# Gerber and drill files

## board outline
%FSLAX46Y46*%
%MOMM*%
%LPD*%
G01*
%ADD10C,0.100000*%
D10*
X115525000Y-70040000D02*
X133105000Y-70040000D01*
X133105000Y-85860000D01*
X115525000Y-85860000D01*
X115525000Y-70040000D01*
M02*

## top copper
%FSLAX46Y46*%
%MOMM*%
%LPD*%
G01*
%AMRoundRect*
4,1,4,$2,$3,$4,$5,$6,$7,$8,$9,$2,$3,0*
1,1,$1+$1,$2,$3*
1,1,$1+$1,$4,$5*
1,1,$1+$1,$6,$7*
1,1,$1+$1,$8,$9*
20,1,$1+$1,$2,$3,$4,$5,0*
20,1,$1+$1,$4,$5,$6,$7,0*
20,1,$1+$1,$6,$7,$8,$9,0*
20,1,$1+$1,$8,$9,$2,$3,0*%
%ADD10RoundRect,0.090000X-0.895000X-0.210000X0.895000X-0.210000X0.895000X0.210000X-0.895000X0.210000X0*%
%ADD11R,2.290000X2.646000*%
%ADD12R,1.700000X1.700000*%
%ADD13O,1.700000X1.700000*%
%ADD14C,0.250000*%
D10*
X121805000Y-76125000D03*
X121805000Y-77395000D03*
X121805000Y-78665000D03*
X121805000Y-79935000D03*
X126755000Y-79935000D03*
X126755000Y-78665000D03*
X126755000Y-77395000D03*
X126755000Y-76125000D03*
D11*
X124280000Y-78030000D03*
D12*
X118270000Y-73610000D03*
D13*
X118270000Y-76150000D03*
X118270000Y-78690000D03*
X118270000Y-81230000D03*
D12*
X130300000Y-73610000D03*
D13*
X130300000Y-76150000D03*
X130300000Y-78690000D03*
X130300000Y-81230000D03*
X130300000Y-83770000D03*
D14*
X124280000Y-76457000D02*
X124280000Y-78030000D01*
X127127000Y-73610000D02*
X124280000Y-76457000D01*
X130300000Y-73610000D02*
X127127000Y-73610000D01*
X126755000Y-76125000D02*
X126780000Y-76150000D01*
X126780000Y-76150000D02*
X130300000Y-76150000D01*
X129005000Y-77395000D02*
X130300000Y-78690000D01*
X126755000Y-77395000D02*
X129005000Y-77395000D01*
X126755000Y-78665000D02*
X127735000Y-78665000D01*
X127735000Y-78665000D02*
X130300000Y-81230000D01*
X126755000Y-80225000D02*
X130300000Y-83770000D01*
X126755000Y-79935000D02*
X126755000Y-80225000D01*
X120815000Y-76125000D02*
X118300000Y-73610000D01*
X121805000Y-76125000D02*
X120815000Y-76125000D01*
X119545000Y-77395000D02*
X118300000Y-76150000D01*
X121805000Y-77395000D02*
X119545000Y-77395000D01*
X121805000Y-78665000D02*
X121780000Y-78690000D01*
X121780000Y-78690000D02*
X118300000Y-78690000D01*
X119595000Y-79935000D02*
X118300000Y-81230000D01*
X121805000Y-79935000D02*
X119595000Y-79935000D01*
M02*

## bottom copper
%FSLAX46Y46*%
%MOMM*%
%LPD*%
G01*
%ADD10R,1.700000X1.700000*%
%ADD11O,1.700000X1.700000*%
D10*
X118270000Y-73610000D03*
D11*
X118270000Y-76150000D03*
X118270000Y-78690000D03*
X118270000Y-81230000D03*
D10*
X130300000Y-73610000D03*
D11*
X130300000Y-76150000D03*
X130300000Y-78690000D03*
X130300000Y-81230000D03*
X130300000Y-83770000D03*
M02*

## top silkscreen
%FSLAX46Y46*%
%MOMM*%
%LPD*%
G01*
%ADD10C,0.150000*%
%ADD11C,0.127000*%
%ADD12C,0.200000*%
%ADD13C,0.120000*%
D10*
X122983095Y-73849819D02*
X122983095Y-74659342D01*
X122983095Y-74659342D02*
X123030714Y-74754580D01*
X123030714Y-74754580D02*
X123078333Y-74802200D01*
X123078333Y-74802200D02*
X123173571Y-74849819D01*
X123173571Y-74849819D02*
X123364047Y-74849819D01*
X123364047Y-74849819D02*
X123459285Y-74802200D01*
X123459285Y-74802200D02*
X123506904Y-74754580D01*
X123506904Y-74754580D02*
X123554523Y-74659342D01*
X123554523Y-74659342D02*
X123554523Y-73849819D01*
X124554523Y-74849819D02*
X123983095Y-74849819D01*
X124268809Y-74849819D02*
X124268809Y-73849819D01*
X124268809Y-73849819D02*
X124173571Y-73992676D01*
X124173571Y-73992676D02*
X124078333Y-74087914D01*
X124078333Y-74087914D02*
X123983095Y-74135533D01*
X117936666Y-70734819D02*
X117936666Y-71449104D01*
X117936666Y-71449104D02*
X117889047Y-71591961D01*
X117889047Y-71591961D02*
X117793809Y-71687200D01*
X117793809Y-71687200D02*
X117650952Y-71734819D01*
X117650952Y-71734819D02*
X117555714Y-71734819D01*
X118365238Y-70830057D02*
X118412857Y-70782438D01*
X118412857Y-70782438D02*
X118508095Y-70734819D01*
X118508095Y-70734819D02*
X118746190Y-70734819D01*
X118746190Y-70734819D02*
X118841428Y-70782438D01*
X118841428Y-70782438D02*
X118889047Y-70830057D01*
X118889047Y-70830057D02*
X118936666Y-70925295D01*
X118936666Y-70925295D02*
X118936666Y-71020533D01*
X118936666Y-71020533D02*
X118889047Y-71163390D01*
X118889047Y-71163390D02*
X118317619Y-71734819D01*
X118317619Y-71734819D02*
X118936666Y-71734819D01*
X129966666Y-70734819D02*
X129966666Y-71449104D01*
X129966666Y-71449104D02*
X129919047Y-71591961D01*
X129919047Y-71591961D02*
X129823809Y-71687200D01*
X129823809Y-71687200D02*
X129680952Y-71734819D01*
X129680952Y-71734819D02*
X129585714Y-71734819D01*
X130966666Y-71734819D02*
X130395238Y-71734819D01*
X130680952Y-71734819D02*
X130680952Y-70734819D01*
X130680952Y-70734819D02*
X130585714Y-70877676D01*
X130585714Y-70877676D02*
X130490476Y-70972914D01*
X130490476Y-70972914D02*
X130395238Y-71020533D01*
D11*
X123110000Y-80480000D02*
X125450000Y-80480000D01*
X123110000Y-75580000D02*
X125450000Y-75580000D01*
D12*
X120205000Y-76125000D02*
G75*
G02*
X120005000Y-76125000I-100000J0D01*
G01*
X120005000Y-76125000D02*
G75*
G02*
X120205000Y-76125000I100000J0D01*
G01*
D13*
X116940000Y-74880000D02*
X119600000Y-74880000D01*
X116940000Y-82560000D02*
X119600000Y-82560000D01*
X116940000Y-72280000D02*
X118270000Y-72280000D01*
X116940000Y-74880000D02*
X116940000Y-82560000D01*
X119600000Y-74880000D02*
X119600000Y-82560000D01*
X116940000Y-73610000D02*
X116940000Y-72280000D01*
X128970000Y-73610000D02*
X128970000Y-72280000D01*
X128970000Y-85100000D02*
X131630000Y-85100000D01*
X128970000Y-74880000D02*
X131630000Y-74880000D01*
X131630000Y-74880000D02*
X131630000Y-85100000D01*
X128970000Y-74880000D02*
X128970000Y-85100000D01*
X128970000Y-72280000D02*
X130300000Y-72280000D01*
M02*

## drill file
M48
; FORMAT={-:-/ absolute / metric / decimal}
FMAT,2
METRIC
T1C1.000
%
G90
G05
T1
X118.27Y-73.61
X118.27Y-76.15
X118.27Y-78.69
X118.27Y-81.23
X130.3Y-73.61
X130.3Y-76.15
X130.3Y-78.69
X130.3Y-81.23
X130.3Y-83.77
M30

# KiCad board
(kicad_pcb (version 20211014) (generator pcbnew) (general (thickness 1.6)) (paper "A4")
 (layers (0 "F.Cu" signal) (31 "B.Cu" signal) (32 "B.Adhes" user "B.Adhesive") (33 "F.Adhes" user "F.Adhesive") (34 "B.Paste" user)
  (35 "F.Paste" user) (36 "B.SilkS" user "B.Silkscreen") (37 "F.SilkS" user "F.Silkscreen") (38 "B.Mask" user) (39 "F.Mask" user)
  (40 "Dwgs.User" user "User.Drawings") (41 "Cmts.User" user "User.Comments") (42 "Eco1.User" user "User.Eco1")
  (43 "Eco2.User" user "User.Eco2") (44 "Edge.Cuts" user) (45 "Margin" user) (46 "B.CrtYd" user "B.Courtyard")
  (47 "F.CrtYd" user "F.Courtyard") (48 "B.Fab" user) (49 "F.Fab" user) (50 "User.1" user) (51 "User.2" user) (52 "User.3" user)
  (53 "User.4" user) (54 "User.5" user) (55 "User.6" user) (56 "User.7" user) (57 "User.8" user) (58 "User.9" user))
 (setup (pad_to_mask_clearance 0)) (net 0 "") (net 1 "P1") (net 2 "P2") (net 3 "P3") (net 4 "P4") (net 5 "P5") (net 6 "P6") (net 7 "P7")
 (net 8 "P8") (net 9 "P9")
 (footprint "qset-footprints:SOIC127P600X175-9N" (layer "F.Cu") (at 124.28 78.03)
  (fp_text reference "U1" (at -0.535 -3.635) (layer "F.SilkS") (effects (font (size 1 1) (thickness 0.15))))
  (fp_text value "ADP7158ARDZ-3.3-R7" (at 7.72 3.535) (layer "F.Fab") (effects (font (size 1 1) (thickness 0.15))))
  (fp_line (start -1.17 2.45) (end 1.17 2.45) (layer "F.SilkS") (width 0.127))
  (fp_line (start -1.17 -2.45) (end 1.17 -2.45) (layer "F.SilkS") (width 0.127))
  (fp_circle (center -4.175 -1.905) (end -4.075 -1.905) (layer "F.SilkS") (width 0.2) (fill none))
  (pad "1" smd roundrect locked (at -2.475 -1.905) (size 1.97 0.6) (layers "F.Cu" "F.Paste" "F.Mask") (roundrect_rratio 0.15) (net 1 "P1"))
  (pad "2" smd roundrect locked (at -2.475 -0.635) (size 1.97 0.6) (layers "F.Cu" "F.Paste" "F.Mask") (roundrect_rratio 0.15) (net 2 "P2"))
  (pad "3" smd roundrect locked (at -2.475 0.635) (size 1.97 0.6) (layers "F.Cu" "F.Paste" "F.Mask") (roundrect_rratio 0.15) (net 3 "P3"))
  (pad "4" smd roundrect locked (at -2.475 1.905) (size 1.97 0.6) (layers "F.Cu" "F.Paste" "F.Mask") (roundrect_rratio 0.15) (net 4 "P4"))
  (pad "5" smd roundrect locked (at 2.475 1.905) (size 1.97 0.6) (layers "F.Cu" "F.Paste" "F.Mask") (roundrect_rratio 0.15) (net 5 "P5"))
  (pad "6" smd roundrect locked (at 2.475 0.635) (size 1.97 0.6) (layers "F.Cu" "F.Paste" "F.Mask") (roundrect_rratio 0.15) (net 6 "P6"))
  (pad "7" smd roundrect locked (at 2.475 -0.635) (size 1.97 0.6) (layers "F.Cu" "F.Paste" "F.Mask") (roundrect_rratio 0.15) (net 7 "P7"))
  (pad "8" smd roundrect locked (at 2.475 -1.905) (size 1.97 0.6) (layers "F.Cu" "F.Paste" "F.Mask") (roundrect_rratio 0.15) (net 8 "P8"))
  (pad "9" smd rect locked (at 0 0) (size 2.29 2.646) (layers "F.Cu" "F.Paste" "F.Mask") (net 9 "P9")))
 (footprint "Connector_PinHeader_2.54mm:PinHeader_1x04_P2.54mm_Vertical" (layer "F.Cu") (at 118.27 73.61)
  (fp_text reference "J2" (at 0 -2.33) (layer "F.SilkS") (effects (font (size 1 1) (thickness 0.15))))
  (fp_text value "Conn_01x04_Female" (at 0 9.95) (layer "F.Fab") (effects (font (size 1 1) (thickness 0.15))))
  (fp_line (start -1.33 1.27) (end 1.33 1.27) (layer "F.SilkS") (width 0.12))
  (fp_line (start -1.33 8.95) (end 1.33 8.95) (layer "F.SilkS") (width 0.12))
  (fp_line (start -1.33 -1.33) (end 0 -1.33) (layer "F.SilkS") (width 0.12))
  (fp_line (start -1.33 1.27) (end -1.33 8.95) (layer "F.SilkS") (width 0.12))
  (fp_line (start 1.33 1.27) (end 1.33 8.95) (layer "F.SilkS") (width 0.12))
  (fp_line (start -1.33 0) (end -1.33 -1.33) (layer "F.SilkS") (width 0.12))
  (pad "1" thru_hole rect (at 0 0) (size 1.7 1.7) (drill 1) (layers *.Cu *.Mask) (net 1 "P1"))
  (pad "2" thru_hole oval (at 0 2.54) (size 1.7 1.7) (drill 1) (layers *.Cu *.Mask) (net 2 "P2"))
  (pad "3" thru_hole oval (at 0 5.08) (size 1.7 1.7) (drill 1) (layers *.Cu *.Mask) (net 3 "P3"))
  (pad "4" thru_hole oval (at 0 7.62) (size 1.7 1.7) (drill 1) (layers *.Cu *.Mask) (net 4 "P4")))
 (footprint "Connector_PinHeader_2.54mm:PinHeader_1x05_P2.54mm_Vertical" (layer "F.Cu") (at 130.3 73.61)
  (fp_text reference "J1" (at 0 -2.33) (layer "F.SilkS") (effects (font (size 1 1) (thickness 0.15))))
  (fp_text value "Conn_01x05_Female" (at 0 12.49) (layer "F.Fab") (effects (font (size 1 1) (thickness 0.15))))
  (fp_line (start -1.33 0) (end -1.33 -1.33) (layer "F.SilkS") (width 0.12))
  (fp_line (start -1.33 11.49) (end 1.33 11.49) (layer "F.SilkS") (width 0.12))
  (fp_line (start -1.33 1.27) (end 1.33 1.27) (layer "F.SilkS") (width 0.12))
  (fp_line (start 1.33 1.27) (end 1.33 11.49) (layer "F.SilkS") (width 0.12))
  (fp_line (start -1.33 1.27) (end -1.33 11.49) (layer "F.SilkS") (width 0.12))
  (fp_line (start -1.33 -1.33) (end 0 -1.33) (layer "F.SilkS") (width 0.12))
  (pad "1" thru_hole rect (at 0 0) (size 1.7 1.7) (drill 1) (layers *.Cu *.Mask) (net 9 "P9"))
  (pad "2" thru_hole oval (at 0 2.54) (size 1.7 1.7) (drill 1) (layers *.Cu *.Mask) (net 8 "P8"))
  (pad "3" thru_hole oval (at 0 5.08) (size 1.7 1.7) (drill 1) (layers *.Cu *.Mask) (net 7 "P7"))
  (pad "4" thru_hole oval (at 0 7.62) (size 1.7 1.7) (drill 1) (layers *.Cu *.Mask) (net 6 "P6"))
  (pad "5" thru_hole oval (at 0 10.16) (size 1.7 1.7) (drill 1) (layers *.Cu *.Mask) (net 5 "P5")))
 (gr_rect (start 115.525 70.04) (end 133.105 85.86) (layer "Edge.Cuts") (width 0.1) (fill none))
 (segment (start 124.28 76.457) (end 124.28 78.03) (width 0.25) (layer "F.Cu") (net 9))
 (segment (start 127.127 73.61) (end 124.28 76.457) (width 0.25) (layer "F.Cu") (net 9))
 (segment (start 130.3 73.61) (end 127.127 73.61) (width 0.25) (layer "F.Cu") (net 9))
 (segment (start 126.755 76.125) (end 126.78 76.15) (width 0.25) (layer "F.Cu") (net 8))
 (segment (start 126.78 76.15) (end 130.3 76.15) (width 0.25) (layer "F.Cu") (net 8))
 (segment (start 129.005 77.395) (end 130.3 78.69) (width 0.25) (layer "F.Cu") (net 7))
 (segment (start 126.755 77.395) (end 129.005 77.395) (width 0.25) (layer "F.Cu") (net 7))
 (segment (start 126.755 78.665) (end 127.735 78.665) (width 0.25) (layer "F.Cu") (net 6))
 (segment (start 127.735 78.665) (end 130.3 81.23) (width 0.25) (layer "F.Cu") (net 6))
 (segment (start 126.755 80.225) (end 130.3 83.77) (width 0.25) (layer "F.Cu") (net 5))
 (segment (start 126.755 79.935) (end 126.755 80.225) (width 0.25) (layer "F.Cu") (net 5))
 (segment (start 120.815 76.125) (end 118.3 73.61) (width 0.25) (layer "F.Cu") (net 1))
 (segment (start 121.805 76.125) (end 120.815 76.125) (width 0.25) (layer "F.Cu") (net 1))
 (segment (start 119.545 77.395) (end 118.3 76.15) (width 0.25) (layer "F.Cu") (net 2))
 (segment (start 121.805 77.395) (end 119.545 77.395) (width 0.25) (layer "F.Cu") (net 2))
 (segment (start 121.805 78.665) (end 121.78 78.69) (width 0.25) (layer "F.Cu") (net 3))
 (segment (start 121.78 78.69) (end 118.3 78.69) (width 0.25) (layer "F.Cu") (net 3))
 (segment (start 119.595 79.935) (end 118.3 81.23) (width 0.25) (layer "F.Cu") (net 4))
 (segment (start 121.805 79.935) (end 119.595 79.935) (width 0.25) (layer "F.Cu") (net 4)))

